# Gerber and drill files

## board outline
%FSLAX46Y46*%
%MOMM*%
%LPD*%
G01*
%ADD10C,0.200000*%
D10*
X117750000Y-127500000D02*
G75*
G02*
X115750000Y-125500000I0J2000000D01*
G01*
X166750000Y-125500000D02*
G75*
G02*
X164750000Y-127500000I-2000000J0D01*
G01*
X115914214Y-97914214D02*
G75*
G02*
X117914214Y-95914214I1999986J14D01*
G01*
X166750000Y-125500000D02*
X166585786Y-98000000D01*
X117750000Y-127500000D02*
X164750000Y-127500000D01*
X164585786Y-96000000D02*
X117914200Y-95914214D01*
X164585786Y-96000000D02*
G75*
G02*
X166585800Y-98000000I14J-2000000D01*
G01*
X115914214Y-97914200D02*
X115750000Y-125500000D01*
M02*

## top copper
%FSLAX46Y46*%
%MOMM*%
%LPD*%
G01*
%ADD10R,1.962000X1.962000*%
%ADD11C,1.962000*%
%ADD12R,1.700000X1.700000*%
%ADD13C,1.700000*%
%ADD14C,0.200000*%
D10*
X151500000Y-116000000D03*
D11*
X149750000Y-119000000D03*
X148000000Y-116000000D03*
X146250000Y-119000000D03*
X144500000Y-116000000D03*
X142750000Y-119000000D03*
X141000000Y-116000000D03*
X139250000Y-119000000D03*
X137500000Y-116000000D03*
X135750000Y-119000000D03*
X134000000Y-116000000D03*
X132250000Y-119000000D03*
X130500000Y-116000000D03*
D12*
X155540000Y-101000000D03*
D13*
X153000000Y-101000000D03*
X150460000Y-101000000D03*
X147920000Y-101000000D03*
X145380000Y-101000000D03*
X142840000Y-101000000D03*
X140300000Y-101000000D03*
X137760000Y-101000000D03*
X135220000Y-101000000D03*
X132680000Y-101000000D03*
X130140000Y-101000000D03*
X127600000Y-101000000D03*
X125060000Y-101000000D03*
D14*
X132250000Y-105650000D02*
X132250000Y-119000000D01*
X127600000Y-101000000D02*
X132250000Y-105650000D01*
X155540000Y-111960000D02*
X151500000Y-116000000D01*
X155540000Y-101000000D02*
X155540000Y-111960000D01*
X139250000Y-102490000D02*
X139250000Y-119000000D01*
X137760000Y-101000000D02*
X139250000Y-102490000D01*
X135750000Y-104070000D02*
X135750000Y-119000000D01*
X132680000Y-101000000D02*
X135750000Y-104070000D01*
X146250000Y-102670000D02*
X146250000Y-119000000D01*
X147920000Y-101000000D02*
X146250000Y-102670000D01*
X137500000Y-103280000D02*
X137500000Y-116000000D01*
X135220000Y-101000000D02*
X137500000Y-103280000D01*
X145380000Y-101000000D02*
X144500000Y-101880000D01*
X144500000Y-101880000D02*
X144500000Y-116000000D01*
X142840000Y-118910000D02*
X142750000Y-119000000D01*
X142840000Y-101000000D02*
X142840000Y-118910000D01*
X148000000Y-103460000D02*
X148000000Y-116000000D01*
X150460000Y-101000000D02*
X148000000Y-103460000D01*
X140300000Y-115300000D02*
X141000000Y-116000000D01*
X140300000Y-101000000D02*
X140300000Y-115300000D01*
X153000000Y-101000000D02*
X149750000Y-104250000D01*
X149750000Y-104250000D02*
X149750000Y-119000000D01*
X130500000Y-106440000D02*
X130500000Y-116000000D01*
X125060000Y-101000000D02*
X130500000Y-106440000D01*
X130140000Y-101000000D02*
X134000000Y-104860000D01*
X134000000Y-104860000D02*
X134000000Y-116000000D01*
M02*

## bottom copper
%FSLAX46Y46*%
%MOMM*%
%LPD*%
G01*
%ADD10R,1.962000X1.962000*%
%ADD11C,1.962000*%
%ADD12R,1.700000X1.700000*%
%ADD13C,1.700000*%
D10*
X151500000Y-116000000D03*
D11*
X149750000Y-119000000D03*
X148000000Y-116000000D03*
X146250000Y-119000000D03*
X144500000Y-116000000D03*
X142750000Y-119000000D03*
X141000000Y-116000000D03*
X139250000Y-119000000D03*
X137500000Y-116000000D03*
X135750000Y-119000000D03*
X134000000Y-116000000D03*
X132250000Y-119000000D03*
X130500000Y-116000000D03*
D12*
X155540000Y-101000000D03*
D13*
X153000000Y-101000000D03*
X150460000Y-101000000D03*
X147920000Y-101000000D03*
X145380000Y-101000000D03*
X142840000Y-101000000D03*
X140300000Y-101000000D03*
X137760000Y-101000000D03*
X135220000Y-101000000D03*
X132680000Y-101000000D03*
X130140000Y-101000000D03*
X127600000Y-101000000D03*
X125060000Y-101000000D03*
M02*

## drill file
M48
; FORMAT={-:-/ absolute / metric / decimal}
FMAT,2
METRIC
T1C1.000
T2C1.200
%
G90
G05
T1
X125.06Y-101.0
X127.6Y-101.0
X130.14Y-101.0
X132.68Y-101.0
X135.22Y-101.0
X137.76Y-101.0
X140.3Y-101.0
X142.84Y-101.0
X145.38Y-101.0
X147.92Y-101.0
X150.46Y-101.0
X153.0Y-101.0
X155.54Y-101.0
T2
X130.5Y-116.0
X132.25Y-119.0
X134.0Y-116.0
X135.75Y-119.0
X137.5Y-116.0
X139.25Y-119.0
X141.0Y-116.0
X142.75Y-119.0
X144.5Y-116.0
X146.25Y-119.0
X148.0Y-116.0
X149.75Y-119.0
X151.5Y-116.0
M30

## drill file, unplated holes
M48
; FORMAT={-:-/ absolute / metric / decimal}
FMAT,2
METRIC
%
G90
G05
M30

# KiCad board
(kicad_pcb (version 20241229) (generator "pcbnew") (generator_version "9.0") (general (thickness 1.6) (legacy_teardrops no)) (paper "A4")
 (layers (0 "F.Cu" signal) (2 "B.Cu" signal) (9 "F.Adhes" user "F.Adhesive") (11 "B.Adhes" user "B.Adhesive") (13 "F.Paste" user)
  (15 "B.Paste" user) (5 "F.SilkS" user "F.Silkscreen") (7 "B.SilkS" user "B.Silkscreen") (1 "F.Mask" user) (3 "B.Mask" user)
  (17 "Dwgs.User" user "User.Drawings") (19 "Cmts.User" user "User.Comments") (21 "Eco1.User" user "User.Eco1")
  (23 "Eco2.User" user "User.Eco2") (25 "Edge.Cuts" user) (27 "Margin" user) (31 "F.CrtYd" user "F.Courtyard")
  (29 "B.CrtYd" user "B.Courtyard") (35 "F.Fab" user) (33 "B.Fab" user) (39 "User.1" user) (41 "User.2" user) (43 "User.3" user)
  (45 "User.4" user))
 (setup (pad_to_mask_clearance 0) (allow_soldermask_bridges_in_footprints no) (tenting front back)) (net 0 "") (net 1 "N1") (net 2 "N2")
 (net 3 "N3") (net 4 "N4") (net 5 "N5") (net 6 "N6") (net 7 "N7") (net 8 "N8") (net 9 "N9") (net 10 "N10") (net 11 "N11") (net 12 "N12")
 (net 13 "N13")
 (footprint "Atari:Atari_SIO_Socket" (layer "F.Cu") (at 142.75 111.5 180)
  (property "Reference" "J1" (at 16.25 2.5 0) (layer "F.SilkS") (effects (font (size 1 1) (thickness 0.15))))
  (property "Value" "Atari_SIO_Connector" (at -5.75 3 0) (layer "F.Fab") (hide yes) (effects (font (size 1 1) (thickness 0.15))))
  (pad "1" thru_hole rect (at -8.75 -4.5 180) (size 1.962 1.962) (drill 1.2) (layers "*.Cu" "*.Mask") (remove_unused_layers no) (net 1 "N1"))
  (pad "2" thru_hole circle (at -7 -7.5 180) (size 1.962 1.962) (drill 1.2) (layers "*.Cu" "*.Mask") (remove_unused_layers no) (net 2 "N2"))
  (pad "3" thru_hole circle (at -5.25 -4.5 180) (size 1.962 1.962) (drill 1.2) (layers "*.Cu" "*.Mask") (remove_unused_layers no)
   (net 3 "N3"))
  (pad "4" thru_hole circle (at -3.5 -7.5 180) (size 1.962 1.962) (drill 1.2) (layers "*.Cu" "*.Mask") (remove_unused_layers no)
   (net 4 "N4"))
  (pad "5" thru_hole circle (at -1.75 -4.5 180) (size 1.962 1.962) (drill 1.2) (layers "*.Cu" "*.Mask") (remove_unused_layers no)
   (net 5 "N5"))
  (pad "6" thru_hole circle (at 0 -7.5 180) (size 1.962 1.962) (drill 1.2) (layers "*.Cu" "*.Mask") (remove_unused_layers no) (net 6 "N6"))
  (pad "7" thru_hole circle (at 1.75 -4.5 180) (size 1.962 1.962) (drill 1.2) (layers "*.Cu" "*.Mask") (remove_unused_layers no)
   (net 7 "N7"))
  (pad "8" thru_hole circle (at 3.5 -7.5 180) (size 1.962 1.962) (drill 1.2) (layers "*.Cu" "*.Mask") (remove_unused_layers no) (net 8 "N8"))
  (pad "9" thru_hole circle (at 5.25 -4.5 180) (size 1.962 1.962) (drill 1.2) (layers "*.Cu" "*.Mask") (remove_unused_layers no)
   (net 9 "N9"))
  (pad "10" thru_hole circle (at 7 -7.5 180) (size 1.962 1.962) (drill 1.2) (layers "*.Cu" "*.Mask") (remove_unused_layers no)
   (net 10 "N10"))
  (pad "11" thru_hole circle (at 8.75 -4.5 180) (size 1.962 1.962) (drill 1.2) (layers "*.Cu" "*.Mask") (remove_unused_layers no)
   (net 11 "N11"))
  (pad "12" thru_hole circle (at 10.5 -7.5 180) (size 1.962 1.962) (drill 1.2) (layers "*.Cu" "*.Mask") (remove_unused_layers no)
   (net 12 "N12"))
  (pad "13" thru_hole circle (at 12.25 -4.5 180) (size 1.962 1.962) (drill 1.2) (layers "*.Cu" "*.Mask") (remove_unused_layers no)
   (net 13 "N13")))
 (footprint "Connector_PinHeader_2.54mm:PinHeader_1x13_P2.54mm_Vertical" (layer "B.Cu") (at 155.54 101 90)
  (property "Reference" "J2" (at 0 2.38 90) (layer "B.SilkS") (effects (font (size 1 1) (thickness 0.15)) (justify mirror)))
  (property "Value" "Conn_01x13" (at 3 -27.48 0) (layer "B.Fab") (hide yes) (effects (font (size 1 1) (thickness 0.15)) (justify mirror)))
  (pad "1" thru_hole rect (at 0 0 90) (size 1.7 1.7) (drill 1) (layers "*.Cu" "*.Mask") (remove_unused_layers no) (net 1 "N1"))
  (pad "2" thru_hole circle (at 0 -2.54 90) (size 1.7 1.7) (drill 1) (layers "*.Cu" "*.Mask") (remove_unused_layers no) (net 2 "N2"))
  (pad "3" thru_hole circle (at 0 -5.08 90) (size 1.7 1.7) (drill 1) (layers "*.Cu" "*.Mask") (remove_unused_layers no) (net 3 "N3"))
  (pad "4" thru_hole circle (at 0 -7.62 90) (size 1.7 1.7) (drill 1) (layers "*.Cu" "*.Mask") (remove_unused_layers no) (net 4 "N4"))
  (pad "5" thru_hole circle (at 0 -10.16 90) (size 1.7 1.7) (drill 1) (layers "*.Cu" "*.Mask") (remove_unused_layers no) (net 5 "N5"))
  (pad "6" thru_hole circle (at 0 -12.7 90) (size 1.7 1.7) (drill 1) (layers "*.Cu" "*.Mask") (remove_unused_layers no) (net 6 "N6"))
  (pad "7" thru_hole circle (at 0 -15.24 90) (size 1.7 1.7) (drill 1) (layers "*.Cu" "*.Mask") (remove_unused_layers no) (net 7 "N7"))
  (pad "8" thru_hole circle (at 0 -17.78 90) (size 1.7 1.7) (drill 1) (layers "*.Cu" "*.Mask") (remove_unused_layers no) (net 8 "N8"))
  (pad "9" thru_hole circle (at 0 -20.32 90) (size 1.7 1.7) (drill 1) (layers "*.Cu" "*.Mask") (remove_unused_layers no) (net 9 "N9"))
  (pad "10" thru_hole circle (at 0 -22.86 90) (size 1.7 1.7) (drill 1) (layers "*.Cu" "*.Mask") (remove_unused_layers no) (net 10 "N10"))
  (pad "11" thru_hole circle (at 0 -25.4 90) (size 1.7 1.7) (drill 1) (layers "*.Cu" "*.Mask") (remove_unused_layers no) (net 11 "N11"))
  (pad "12" thru_hole circle (at 0 -27.94 90) (size 1.7 1.7) (drill 1) (layers "*.Cu" "*.Mask") (remove_unused_layers no) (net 12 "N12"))
  (pad "13" thru_hole circle (at 0 -30.48 90) (size 1.7 1.7) (drill 1) (layers "*.Cu" "*.Mask") (remove_unused_layers no) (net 13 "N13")))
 (gr_arc (start 117.75 127.5) (mid 116.335786 126.914214) (end 115.75 125.5) (stroke (width 0.2) (type solid)) (layer "Edge.Cuts"))
 (gr_arc (start 166.75 125.5) (mid 166.164214 126.914214) (end 164.75 127.5) (stroke (width 0.2) (type solid)) (layer "Edge.Cuts"))
 (gr_arc (start 115.914214 97.914214) (mid 116.5 96.5) (end 117.914214 95.914214) (stroke (width 0.2) (type solid)) (layer "Edge.Cuts"))
 (gr_line (start 166.75 125.5) (end 166.585786 98) (stroke (width 0.2) (type solid)) (layer "Edge.Cuts"))
 (gr_line (start 117.75 127.5) (end 164.75 127.5) (stroke (width 0.2) (type solid)) (layer "Edge.Cuts"))
 (gr_line (start 164.585786 96) (end 117.9142 95.914214) (stroke (width 0.2) (type solid)) (layer "Edge.Cuts"))
 (gr_arc (start 164.585786 96) (mid 166 96.585786) (end 166.585786 98) (stroke (width 0.2) (type solid)) (layer "Edge.Cuts"))
 (gr_line (start 115.914214 97.9142) (end 115.75 125.5) (stroke (width 0.2) (type solid)) (layer "Edge.Cuts"))
 (segment (start 132.25 105.65) (end 132.25 119) (width 0.2) (layer "F.Cu") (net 12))
 (segment (start 127.6 101) (end 132.25 105.65) (width 0.2) (layer "F.Cu") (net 12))
 (segment (start 155.54 111.96) (end 151.5 116) (width 0.2) (layer "F.Cu") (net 1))
 (segment (start 155.54 101) (end 155.54 111.96) (width 0.2) (layer "F.Cu") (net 1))
 (segment (start 139.25 102.49) (end 139.25 119) (width 0.2) (layer "F.Cu") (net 8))
 (segment (start 137.76 101) (end 139.25 102.49) (width 0.2) (layer "F.Cu") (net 8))
 (segment (start 135.75 104.07) (end 135.75 119) (width 0.2) (layer "F.Cu") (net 10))
 (segment (start 132.68 101) (end 135.75 104.07) (width 0.2) (layer "F.Cu") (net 10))
 (segment (start 146.25 102.67) (end 146.25 119) (width 0.2) (layer "F.Cu") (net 4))
 (segment (start 147.92 101) (end 146.25 102.67) (width 0.2) (layer "F.Cu") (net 4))
 (segment (start 137.5 103.28) (end 137.5 116) (width 0.2) (layer "F.Cu") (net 9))
 (segment (start 135.22 101) (end 137.5 103.28) (width 0.2) (layer "F.Cu") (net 9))
 (segment (start 145.38 101) (end 144.5 101.88) (width 0.2) (layer "F.Cu") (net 5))
 (segment (start 144.5 101.88) (end 144.5 116) (width 0.2) (layer "F.Cu") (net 5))
 (segment (start 142.84 118.91) (end 142.75 119) (width 0.2) (layer "F.Cu") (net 6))
 (segment (start 142.84 101) (end 142.84 118.91) (width 0.2) (layer "F.Cu") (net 6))
 (segment (start 148 103.46) (end 148 116) (width 0.2) (layer "F.Cu") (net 3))
 (segment (start 150.46 101) (end 148 103.46) (width 0.2) (layer "F.Cu") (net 3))
 (segment (start 140.3 115.3) (end 141 116) (width 0.2) (layer "F.Cu") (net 7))
 (segment (start 140.3 101) (end 140.3 115.3) (width 0.2) (layer "F.Cu") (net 7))
 (segment (start 153 101) (end 149.75 104.25) (width 0.2) (layer "F.Cu") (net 2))
 (segment (start 149.75 104.25) (end 149.75 119) (width 0.2) (layer "F.Cu") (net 2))
 (segment (start 130.5 106.44) (end 130.5 116) (width 0.2) (layer "F.Cu") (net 13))
 (segment (start 125.06 101) (end 130.5 106.44) (width 0.2) (layer "F.Cu") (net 13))
 (segment (start 130.14 101) (end 134 104.86) (width 0.2) (layer "F.Cu") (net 11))
 (segment (start 134 104.86) (end 134 116) (width 0.2) (layer "F.Cu") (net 11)))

